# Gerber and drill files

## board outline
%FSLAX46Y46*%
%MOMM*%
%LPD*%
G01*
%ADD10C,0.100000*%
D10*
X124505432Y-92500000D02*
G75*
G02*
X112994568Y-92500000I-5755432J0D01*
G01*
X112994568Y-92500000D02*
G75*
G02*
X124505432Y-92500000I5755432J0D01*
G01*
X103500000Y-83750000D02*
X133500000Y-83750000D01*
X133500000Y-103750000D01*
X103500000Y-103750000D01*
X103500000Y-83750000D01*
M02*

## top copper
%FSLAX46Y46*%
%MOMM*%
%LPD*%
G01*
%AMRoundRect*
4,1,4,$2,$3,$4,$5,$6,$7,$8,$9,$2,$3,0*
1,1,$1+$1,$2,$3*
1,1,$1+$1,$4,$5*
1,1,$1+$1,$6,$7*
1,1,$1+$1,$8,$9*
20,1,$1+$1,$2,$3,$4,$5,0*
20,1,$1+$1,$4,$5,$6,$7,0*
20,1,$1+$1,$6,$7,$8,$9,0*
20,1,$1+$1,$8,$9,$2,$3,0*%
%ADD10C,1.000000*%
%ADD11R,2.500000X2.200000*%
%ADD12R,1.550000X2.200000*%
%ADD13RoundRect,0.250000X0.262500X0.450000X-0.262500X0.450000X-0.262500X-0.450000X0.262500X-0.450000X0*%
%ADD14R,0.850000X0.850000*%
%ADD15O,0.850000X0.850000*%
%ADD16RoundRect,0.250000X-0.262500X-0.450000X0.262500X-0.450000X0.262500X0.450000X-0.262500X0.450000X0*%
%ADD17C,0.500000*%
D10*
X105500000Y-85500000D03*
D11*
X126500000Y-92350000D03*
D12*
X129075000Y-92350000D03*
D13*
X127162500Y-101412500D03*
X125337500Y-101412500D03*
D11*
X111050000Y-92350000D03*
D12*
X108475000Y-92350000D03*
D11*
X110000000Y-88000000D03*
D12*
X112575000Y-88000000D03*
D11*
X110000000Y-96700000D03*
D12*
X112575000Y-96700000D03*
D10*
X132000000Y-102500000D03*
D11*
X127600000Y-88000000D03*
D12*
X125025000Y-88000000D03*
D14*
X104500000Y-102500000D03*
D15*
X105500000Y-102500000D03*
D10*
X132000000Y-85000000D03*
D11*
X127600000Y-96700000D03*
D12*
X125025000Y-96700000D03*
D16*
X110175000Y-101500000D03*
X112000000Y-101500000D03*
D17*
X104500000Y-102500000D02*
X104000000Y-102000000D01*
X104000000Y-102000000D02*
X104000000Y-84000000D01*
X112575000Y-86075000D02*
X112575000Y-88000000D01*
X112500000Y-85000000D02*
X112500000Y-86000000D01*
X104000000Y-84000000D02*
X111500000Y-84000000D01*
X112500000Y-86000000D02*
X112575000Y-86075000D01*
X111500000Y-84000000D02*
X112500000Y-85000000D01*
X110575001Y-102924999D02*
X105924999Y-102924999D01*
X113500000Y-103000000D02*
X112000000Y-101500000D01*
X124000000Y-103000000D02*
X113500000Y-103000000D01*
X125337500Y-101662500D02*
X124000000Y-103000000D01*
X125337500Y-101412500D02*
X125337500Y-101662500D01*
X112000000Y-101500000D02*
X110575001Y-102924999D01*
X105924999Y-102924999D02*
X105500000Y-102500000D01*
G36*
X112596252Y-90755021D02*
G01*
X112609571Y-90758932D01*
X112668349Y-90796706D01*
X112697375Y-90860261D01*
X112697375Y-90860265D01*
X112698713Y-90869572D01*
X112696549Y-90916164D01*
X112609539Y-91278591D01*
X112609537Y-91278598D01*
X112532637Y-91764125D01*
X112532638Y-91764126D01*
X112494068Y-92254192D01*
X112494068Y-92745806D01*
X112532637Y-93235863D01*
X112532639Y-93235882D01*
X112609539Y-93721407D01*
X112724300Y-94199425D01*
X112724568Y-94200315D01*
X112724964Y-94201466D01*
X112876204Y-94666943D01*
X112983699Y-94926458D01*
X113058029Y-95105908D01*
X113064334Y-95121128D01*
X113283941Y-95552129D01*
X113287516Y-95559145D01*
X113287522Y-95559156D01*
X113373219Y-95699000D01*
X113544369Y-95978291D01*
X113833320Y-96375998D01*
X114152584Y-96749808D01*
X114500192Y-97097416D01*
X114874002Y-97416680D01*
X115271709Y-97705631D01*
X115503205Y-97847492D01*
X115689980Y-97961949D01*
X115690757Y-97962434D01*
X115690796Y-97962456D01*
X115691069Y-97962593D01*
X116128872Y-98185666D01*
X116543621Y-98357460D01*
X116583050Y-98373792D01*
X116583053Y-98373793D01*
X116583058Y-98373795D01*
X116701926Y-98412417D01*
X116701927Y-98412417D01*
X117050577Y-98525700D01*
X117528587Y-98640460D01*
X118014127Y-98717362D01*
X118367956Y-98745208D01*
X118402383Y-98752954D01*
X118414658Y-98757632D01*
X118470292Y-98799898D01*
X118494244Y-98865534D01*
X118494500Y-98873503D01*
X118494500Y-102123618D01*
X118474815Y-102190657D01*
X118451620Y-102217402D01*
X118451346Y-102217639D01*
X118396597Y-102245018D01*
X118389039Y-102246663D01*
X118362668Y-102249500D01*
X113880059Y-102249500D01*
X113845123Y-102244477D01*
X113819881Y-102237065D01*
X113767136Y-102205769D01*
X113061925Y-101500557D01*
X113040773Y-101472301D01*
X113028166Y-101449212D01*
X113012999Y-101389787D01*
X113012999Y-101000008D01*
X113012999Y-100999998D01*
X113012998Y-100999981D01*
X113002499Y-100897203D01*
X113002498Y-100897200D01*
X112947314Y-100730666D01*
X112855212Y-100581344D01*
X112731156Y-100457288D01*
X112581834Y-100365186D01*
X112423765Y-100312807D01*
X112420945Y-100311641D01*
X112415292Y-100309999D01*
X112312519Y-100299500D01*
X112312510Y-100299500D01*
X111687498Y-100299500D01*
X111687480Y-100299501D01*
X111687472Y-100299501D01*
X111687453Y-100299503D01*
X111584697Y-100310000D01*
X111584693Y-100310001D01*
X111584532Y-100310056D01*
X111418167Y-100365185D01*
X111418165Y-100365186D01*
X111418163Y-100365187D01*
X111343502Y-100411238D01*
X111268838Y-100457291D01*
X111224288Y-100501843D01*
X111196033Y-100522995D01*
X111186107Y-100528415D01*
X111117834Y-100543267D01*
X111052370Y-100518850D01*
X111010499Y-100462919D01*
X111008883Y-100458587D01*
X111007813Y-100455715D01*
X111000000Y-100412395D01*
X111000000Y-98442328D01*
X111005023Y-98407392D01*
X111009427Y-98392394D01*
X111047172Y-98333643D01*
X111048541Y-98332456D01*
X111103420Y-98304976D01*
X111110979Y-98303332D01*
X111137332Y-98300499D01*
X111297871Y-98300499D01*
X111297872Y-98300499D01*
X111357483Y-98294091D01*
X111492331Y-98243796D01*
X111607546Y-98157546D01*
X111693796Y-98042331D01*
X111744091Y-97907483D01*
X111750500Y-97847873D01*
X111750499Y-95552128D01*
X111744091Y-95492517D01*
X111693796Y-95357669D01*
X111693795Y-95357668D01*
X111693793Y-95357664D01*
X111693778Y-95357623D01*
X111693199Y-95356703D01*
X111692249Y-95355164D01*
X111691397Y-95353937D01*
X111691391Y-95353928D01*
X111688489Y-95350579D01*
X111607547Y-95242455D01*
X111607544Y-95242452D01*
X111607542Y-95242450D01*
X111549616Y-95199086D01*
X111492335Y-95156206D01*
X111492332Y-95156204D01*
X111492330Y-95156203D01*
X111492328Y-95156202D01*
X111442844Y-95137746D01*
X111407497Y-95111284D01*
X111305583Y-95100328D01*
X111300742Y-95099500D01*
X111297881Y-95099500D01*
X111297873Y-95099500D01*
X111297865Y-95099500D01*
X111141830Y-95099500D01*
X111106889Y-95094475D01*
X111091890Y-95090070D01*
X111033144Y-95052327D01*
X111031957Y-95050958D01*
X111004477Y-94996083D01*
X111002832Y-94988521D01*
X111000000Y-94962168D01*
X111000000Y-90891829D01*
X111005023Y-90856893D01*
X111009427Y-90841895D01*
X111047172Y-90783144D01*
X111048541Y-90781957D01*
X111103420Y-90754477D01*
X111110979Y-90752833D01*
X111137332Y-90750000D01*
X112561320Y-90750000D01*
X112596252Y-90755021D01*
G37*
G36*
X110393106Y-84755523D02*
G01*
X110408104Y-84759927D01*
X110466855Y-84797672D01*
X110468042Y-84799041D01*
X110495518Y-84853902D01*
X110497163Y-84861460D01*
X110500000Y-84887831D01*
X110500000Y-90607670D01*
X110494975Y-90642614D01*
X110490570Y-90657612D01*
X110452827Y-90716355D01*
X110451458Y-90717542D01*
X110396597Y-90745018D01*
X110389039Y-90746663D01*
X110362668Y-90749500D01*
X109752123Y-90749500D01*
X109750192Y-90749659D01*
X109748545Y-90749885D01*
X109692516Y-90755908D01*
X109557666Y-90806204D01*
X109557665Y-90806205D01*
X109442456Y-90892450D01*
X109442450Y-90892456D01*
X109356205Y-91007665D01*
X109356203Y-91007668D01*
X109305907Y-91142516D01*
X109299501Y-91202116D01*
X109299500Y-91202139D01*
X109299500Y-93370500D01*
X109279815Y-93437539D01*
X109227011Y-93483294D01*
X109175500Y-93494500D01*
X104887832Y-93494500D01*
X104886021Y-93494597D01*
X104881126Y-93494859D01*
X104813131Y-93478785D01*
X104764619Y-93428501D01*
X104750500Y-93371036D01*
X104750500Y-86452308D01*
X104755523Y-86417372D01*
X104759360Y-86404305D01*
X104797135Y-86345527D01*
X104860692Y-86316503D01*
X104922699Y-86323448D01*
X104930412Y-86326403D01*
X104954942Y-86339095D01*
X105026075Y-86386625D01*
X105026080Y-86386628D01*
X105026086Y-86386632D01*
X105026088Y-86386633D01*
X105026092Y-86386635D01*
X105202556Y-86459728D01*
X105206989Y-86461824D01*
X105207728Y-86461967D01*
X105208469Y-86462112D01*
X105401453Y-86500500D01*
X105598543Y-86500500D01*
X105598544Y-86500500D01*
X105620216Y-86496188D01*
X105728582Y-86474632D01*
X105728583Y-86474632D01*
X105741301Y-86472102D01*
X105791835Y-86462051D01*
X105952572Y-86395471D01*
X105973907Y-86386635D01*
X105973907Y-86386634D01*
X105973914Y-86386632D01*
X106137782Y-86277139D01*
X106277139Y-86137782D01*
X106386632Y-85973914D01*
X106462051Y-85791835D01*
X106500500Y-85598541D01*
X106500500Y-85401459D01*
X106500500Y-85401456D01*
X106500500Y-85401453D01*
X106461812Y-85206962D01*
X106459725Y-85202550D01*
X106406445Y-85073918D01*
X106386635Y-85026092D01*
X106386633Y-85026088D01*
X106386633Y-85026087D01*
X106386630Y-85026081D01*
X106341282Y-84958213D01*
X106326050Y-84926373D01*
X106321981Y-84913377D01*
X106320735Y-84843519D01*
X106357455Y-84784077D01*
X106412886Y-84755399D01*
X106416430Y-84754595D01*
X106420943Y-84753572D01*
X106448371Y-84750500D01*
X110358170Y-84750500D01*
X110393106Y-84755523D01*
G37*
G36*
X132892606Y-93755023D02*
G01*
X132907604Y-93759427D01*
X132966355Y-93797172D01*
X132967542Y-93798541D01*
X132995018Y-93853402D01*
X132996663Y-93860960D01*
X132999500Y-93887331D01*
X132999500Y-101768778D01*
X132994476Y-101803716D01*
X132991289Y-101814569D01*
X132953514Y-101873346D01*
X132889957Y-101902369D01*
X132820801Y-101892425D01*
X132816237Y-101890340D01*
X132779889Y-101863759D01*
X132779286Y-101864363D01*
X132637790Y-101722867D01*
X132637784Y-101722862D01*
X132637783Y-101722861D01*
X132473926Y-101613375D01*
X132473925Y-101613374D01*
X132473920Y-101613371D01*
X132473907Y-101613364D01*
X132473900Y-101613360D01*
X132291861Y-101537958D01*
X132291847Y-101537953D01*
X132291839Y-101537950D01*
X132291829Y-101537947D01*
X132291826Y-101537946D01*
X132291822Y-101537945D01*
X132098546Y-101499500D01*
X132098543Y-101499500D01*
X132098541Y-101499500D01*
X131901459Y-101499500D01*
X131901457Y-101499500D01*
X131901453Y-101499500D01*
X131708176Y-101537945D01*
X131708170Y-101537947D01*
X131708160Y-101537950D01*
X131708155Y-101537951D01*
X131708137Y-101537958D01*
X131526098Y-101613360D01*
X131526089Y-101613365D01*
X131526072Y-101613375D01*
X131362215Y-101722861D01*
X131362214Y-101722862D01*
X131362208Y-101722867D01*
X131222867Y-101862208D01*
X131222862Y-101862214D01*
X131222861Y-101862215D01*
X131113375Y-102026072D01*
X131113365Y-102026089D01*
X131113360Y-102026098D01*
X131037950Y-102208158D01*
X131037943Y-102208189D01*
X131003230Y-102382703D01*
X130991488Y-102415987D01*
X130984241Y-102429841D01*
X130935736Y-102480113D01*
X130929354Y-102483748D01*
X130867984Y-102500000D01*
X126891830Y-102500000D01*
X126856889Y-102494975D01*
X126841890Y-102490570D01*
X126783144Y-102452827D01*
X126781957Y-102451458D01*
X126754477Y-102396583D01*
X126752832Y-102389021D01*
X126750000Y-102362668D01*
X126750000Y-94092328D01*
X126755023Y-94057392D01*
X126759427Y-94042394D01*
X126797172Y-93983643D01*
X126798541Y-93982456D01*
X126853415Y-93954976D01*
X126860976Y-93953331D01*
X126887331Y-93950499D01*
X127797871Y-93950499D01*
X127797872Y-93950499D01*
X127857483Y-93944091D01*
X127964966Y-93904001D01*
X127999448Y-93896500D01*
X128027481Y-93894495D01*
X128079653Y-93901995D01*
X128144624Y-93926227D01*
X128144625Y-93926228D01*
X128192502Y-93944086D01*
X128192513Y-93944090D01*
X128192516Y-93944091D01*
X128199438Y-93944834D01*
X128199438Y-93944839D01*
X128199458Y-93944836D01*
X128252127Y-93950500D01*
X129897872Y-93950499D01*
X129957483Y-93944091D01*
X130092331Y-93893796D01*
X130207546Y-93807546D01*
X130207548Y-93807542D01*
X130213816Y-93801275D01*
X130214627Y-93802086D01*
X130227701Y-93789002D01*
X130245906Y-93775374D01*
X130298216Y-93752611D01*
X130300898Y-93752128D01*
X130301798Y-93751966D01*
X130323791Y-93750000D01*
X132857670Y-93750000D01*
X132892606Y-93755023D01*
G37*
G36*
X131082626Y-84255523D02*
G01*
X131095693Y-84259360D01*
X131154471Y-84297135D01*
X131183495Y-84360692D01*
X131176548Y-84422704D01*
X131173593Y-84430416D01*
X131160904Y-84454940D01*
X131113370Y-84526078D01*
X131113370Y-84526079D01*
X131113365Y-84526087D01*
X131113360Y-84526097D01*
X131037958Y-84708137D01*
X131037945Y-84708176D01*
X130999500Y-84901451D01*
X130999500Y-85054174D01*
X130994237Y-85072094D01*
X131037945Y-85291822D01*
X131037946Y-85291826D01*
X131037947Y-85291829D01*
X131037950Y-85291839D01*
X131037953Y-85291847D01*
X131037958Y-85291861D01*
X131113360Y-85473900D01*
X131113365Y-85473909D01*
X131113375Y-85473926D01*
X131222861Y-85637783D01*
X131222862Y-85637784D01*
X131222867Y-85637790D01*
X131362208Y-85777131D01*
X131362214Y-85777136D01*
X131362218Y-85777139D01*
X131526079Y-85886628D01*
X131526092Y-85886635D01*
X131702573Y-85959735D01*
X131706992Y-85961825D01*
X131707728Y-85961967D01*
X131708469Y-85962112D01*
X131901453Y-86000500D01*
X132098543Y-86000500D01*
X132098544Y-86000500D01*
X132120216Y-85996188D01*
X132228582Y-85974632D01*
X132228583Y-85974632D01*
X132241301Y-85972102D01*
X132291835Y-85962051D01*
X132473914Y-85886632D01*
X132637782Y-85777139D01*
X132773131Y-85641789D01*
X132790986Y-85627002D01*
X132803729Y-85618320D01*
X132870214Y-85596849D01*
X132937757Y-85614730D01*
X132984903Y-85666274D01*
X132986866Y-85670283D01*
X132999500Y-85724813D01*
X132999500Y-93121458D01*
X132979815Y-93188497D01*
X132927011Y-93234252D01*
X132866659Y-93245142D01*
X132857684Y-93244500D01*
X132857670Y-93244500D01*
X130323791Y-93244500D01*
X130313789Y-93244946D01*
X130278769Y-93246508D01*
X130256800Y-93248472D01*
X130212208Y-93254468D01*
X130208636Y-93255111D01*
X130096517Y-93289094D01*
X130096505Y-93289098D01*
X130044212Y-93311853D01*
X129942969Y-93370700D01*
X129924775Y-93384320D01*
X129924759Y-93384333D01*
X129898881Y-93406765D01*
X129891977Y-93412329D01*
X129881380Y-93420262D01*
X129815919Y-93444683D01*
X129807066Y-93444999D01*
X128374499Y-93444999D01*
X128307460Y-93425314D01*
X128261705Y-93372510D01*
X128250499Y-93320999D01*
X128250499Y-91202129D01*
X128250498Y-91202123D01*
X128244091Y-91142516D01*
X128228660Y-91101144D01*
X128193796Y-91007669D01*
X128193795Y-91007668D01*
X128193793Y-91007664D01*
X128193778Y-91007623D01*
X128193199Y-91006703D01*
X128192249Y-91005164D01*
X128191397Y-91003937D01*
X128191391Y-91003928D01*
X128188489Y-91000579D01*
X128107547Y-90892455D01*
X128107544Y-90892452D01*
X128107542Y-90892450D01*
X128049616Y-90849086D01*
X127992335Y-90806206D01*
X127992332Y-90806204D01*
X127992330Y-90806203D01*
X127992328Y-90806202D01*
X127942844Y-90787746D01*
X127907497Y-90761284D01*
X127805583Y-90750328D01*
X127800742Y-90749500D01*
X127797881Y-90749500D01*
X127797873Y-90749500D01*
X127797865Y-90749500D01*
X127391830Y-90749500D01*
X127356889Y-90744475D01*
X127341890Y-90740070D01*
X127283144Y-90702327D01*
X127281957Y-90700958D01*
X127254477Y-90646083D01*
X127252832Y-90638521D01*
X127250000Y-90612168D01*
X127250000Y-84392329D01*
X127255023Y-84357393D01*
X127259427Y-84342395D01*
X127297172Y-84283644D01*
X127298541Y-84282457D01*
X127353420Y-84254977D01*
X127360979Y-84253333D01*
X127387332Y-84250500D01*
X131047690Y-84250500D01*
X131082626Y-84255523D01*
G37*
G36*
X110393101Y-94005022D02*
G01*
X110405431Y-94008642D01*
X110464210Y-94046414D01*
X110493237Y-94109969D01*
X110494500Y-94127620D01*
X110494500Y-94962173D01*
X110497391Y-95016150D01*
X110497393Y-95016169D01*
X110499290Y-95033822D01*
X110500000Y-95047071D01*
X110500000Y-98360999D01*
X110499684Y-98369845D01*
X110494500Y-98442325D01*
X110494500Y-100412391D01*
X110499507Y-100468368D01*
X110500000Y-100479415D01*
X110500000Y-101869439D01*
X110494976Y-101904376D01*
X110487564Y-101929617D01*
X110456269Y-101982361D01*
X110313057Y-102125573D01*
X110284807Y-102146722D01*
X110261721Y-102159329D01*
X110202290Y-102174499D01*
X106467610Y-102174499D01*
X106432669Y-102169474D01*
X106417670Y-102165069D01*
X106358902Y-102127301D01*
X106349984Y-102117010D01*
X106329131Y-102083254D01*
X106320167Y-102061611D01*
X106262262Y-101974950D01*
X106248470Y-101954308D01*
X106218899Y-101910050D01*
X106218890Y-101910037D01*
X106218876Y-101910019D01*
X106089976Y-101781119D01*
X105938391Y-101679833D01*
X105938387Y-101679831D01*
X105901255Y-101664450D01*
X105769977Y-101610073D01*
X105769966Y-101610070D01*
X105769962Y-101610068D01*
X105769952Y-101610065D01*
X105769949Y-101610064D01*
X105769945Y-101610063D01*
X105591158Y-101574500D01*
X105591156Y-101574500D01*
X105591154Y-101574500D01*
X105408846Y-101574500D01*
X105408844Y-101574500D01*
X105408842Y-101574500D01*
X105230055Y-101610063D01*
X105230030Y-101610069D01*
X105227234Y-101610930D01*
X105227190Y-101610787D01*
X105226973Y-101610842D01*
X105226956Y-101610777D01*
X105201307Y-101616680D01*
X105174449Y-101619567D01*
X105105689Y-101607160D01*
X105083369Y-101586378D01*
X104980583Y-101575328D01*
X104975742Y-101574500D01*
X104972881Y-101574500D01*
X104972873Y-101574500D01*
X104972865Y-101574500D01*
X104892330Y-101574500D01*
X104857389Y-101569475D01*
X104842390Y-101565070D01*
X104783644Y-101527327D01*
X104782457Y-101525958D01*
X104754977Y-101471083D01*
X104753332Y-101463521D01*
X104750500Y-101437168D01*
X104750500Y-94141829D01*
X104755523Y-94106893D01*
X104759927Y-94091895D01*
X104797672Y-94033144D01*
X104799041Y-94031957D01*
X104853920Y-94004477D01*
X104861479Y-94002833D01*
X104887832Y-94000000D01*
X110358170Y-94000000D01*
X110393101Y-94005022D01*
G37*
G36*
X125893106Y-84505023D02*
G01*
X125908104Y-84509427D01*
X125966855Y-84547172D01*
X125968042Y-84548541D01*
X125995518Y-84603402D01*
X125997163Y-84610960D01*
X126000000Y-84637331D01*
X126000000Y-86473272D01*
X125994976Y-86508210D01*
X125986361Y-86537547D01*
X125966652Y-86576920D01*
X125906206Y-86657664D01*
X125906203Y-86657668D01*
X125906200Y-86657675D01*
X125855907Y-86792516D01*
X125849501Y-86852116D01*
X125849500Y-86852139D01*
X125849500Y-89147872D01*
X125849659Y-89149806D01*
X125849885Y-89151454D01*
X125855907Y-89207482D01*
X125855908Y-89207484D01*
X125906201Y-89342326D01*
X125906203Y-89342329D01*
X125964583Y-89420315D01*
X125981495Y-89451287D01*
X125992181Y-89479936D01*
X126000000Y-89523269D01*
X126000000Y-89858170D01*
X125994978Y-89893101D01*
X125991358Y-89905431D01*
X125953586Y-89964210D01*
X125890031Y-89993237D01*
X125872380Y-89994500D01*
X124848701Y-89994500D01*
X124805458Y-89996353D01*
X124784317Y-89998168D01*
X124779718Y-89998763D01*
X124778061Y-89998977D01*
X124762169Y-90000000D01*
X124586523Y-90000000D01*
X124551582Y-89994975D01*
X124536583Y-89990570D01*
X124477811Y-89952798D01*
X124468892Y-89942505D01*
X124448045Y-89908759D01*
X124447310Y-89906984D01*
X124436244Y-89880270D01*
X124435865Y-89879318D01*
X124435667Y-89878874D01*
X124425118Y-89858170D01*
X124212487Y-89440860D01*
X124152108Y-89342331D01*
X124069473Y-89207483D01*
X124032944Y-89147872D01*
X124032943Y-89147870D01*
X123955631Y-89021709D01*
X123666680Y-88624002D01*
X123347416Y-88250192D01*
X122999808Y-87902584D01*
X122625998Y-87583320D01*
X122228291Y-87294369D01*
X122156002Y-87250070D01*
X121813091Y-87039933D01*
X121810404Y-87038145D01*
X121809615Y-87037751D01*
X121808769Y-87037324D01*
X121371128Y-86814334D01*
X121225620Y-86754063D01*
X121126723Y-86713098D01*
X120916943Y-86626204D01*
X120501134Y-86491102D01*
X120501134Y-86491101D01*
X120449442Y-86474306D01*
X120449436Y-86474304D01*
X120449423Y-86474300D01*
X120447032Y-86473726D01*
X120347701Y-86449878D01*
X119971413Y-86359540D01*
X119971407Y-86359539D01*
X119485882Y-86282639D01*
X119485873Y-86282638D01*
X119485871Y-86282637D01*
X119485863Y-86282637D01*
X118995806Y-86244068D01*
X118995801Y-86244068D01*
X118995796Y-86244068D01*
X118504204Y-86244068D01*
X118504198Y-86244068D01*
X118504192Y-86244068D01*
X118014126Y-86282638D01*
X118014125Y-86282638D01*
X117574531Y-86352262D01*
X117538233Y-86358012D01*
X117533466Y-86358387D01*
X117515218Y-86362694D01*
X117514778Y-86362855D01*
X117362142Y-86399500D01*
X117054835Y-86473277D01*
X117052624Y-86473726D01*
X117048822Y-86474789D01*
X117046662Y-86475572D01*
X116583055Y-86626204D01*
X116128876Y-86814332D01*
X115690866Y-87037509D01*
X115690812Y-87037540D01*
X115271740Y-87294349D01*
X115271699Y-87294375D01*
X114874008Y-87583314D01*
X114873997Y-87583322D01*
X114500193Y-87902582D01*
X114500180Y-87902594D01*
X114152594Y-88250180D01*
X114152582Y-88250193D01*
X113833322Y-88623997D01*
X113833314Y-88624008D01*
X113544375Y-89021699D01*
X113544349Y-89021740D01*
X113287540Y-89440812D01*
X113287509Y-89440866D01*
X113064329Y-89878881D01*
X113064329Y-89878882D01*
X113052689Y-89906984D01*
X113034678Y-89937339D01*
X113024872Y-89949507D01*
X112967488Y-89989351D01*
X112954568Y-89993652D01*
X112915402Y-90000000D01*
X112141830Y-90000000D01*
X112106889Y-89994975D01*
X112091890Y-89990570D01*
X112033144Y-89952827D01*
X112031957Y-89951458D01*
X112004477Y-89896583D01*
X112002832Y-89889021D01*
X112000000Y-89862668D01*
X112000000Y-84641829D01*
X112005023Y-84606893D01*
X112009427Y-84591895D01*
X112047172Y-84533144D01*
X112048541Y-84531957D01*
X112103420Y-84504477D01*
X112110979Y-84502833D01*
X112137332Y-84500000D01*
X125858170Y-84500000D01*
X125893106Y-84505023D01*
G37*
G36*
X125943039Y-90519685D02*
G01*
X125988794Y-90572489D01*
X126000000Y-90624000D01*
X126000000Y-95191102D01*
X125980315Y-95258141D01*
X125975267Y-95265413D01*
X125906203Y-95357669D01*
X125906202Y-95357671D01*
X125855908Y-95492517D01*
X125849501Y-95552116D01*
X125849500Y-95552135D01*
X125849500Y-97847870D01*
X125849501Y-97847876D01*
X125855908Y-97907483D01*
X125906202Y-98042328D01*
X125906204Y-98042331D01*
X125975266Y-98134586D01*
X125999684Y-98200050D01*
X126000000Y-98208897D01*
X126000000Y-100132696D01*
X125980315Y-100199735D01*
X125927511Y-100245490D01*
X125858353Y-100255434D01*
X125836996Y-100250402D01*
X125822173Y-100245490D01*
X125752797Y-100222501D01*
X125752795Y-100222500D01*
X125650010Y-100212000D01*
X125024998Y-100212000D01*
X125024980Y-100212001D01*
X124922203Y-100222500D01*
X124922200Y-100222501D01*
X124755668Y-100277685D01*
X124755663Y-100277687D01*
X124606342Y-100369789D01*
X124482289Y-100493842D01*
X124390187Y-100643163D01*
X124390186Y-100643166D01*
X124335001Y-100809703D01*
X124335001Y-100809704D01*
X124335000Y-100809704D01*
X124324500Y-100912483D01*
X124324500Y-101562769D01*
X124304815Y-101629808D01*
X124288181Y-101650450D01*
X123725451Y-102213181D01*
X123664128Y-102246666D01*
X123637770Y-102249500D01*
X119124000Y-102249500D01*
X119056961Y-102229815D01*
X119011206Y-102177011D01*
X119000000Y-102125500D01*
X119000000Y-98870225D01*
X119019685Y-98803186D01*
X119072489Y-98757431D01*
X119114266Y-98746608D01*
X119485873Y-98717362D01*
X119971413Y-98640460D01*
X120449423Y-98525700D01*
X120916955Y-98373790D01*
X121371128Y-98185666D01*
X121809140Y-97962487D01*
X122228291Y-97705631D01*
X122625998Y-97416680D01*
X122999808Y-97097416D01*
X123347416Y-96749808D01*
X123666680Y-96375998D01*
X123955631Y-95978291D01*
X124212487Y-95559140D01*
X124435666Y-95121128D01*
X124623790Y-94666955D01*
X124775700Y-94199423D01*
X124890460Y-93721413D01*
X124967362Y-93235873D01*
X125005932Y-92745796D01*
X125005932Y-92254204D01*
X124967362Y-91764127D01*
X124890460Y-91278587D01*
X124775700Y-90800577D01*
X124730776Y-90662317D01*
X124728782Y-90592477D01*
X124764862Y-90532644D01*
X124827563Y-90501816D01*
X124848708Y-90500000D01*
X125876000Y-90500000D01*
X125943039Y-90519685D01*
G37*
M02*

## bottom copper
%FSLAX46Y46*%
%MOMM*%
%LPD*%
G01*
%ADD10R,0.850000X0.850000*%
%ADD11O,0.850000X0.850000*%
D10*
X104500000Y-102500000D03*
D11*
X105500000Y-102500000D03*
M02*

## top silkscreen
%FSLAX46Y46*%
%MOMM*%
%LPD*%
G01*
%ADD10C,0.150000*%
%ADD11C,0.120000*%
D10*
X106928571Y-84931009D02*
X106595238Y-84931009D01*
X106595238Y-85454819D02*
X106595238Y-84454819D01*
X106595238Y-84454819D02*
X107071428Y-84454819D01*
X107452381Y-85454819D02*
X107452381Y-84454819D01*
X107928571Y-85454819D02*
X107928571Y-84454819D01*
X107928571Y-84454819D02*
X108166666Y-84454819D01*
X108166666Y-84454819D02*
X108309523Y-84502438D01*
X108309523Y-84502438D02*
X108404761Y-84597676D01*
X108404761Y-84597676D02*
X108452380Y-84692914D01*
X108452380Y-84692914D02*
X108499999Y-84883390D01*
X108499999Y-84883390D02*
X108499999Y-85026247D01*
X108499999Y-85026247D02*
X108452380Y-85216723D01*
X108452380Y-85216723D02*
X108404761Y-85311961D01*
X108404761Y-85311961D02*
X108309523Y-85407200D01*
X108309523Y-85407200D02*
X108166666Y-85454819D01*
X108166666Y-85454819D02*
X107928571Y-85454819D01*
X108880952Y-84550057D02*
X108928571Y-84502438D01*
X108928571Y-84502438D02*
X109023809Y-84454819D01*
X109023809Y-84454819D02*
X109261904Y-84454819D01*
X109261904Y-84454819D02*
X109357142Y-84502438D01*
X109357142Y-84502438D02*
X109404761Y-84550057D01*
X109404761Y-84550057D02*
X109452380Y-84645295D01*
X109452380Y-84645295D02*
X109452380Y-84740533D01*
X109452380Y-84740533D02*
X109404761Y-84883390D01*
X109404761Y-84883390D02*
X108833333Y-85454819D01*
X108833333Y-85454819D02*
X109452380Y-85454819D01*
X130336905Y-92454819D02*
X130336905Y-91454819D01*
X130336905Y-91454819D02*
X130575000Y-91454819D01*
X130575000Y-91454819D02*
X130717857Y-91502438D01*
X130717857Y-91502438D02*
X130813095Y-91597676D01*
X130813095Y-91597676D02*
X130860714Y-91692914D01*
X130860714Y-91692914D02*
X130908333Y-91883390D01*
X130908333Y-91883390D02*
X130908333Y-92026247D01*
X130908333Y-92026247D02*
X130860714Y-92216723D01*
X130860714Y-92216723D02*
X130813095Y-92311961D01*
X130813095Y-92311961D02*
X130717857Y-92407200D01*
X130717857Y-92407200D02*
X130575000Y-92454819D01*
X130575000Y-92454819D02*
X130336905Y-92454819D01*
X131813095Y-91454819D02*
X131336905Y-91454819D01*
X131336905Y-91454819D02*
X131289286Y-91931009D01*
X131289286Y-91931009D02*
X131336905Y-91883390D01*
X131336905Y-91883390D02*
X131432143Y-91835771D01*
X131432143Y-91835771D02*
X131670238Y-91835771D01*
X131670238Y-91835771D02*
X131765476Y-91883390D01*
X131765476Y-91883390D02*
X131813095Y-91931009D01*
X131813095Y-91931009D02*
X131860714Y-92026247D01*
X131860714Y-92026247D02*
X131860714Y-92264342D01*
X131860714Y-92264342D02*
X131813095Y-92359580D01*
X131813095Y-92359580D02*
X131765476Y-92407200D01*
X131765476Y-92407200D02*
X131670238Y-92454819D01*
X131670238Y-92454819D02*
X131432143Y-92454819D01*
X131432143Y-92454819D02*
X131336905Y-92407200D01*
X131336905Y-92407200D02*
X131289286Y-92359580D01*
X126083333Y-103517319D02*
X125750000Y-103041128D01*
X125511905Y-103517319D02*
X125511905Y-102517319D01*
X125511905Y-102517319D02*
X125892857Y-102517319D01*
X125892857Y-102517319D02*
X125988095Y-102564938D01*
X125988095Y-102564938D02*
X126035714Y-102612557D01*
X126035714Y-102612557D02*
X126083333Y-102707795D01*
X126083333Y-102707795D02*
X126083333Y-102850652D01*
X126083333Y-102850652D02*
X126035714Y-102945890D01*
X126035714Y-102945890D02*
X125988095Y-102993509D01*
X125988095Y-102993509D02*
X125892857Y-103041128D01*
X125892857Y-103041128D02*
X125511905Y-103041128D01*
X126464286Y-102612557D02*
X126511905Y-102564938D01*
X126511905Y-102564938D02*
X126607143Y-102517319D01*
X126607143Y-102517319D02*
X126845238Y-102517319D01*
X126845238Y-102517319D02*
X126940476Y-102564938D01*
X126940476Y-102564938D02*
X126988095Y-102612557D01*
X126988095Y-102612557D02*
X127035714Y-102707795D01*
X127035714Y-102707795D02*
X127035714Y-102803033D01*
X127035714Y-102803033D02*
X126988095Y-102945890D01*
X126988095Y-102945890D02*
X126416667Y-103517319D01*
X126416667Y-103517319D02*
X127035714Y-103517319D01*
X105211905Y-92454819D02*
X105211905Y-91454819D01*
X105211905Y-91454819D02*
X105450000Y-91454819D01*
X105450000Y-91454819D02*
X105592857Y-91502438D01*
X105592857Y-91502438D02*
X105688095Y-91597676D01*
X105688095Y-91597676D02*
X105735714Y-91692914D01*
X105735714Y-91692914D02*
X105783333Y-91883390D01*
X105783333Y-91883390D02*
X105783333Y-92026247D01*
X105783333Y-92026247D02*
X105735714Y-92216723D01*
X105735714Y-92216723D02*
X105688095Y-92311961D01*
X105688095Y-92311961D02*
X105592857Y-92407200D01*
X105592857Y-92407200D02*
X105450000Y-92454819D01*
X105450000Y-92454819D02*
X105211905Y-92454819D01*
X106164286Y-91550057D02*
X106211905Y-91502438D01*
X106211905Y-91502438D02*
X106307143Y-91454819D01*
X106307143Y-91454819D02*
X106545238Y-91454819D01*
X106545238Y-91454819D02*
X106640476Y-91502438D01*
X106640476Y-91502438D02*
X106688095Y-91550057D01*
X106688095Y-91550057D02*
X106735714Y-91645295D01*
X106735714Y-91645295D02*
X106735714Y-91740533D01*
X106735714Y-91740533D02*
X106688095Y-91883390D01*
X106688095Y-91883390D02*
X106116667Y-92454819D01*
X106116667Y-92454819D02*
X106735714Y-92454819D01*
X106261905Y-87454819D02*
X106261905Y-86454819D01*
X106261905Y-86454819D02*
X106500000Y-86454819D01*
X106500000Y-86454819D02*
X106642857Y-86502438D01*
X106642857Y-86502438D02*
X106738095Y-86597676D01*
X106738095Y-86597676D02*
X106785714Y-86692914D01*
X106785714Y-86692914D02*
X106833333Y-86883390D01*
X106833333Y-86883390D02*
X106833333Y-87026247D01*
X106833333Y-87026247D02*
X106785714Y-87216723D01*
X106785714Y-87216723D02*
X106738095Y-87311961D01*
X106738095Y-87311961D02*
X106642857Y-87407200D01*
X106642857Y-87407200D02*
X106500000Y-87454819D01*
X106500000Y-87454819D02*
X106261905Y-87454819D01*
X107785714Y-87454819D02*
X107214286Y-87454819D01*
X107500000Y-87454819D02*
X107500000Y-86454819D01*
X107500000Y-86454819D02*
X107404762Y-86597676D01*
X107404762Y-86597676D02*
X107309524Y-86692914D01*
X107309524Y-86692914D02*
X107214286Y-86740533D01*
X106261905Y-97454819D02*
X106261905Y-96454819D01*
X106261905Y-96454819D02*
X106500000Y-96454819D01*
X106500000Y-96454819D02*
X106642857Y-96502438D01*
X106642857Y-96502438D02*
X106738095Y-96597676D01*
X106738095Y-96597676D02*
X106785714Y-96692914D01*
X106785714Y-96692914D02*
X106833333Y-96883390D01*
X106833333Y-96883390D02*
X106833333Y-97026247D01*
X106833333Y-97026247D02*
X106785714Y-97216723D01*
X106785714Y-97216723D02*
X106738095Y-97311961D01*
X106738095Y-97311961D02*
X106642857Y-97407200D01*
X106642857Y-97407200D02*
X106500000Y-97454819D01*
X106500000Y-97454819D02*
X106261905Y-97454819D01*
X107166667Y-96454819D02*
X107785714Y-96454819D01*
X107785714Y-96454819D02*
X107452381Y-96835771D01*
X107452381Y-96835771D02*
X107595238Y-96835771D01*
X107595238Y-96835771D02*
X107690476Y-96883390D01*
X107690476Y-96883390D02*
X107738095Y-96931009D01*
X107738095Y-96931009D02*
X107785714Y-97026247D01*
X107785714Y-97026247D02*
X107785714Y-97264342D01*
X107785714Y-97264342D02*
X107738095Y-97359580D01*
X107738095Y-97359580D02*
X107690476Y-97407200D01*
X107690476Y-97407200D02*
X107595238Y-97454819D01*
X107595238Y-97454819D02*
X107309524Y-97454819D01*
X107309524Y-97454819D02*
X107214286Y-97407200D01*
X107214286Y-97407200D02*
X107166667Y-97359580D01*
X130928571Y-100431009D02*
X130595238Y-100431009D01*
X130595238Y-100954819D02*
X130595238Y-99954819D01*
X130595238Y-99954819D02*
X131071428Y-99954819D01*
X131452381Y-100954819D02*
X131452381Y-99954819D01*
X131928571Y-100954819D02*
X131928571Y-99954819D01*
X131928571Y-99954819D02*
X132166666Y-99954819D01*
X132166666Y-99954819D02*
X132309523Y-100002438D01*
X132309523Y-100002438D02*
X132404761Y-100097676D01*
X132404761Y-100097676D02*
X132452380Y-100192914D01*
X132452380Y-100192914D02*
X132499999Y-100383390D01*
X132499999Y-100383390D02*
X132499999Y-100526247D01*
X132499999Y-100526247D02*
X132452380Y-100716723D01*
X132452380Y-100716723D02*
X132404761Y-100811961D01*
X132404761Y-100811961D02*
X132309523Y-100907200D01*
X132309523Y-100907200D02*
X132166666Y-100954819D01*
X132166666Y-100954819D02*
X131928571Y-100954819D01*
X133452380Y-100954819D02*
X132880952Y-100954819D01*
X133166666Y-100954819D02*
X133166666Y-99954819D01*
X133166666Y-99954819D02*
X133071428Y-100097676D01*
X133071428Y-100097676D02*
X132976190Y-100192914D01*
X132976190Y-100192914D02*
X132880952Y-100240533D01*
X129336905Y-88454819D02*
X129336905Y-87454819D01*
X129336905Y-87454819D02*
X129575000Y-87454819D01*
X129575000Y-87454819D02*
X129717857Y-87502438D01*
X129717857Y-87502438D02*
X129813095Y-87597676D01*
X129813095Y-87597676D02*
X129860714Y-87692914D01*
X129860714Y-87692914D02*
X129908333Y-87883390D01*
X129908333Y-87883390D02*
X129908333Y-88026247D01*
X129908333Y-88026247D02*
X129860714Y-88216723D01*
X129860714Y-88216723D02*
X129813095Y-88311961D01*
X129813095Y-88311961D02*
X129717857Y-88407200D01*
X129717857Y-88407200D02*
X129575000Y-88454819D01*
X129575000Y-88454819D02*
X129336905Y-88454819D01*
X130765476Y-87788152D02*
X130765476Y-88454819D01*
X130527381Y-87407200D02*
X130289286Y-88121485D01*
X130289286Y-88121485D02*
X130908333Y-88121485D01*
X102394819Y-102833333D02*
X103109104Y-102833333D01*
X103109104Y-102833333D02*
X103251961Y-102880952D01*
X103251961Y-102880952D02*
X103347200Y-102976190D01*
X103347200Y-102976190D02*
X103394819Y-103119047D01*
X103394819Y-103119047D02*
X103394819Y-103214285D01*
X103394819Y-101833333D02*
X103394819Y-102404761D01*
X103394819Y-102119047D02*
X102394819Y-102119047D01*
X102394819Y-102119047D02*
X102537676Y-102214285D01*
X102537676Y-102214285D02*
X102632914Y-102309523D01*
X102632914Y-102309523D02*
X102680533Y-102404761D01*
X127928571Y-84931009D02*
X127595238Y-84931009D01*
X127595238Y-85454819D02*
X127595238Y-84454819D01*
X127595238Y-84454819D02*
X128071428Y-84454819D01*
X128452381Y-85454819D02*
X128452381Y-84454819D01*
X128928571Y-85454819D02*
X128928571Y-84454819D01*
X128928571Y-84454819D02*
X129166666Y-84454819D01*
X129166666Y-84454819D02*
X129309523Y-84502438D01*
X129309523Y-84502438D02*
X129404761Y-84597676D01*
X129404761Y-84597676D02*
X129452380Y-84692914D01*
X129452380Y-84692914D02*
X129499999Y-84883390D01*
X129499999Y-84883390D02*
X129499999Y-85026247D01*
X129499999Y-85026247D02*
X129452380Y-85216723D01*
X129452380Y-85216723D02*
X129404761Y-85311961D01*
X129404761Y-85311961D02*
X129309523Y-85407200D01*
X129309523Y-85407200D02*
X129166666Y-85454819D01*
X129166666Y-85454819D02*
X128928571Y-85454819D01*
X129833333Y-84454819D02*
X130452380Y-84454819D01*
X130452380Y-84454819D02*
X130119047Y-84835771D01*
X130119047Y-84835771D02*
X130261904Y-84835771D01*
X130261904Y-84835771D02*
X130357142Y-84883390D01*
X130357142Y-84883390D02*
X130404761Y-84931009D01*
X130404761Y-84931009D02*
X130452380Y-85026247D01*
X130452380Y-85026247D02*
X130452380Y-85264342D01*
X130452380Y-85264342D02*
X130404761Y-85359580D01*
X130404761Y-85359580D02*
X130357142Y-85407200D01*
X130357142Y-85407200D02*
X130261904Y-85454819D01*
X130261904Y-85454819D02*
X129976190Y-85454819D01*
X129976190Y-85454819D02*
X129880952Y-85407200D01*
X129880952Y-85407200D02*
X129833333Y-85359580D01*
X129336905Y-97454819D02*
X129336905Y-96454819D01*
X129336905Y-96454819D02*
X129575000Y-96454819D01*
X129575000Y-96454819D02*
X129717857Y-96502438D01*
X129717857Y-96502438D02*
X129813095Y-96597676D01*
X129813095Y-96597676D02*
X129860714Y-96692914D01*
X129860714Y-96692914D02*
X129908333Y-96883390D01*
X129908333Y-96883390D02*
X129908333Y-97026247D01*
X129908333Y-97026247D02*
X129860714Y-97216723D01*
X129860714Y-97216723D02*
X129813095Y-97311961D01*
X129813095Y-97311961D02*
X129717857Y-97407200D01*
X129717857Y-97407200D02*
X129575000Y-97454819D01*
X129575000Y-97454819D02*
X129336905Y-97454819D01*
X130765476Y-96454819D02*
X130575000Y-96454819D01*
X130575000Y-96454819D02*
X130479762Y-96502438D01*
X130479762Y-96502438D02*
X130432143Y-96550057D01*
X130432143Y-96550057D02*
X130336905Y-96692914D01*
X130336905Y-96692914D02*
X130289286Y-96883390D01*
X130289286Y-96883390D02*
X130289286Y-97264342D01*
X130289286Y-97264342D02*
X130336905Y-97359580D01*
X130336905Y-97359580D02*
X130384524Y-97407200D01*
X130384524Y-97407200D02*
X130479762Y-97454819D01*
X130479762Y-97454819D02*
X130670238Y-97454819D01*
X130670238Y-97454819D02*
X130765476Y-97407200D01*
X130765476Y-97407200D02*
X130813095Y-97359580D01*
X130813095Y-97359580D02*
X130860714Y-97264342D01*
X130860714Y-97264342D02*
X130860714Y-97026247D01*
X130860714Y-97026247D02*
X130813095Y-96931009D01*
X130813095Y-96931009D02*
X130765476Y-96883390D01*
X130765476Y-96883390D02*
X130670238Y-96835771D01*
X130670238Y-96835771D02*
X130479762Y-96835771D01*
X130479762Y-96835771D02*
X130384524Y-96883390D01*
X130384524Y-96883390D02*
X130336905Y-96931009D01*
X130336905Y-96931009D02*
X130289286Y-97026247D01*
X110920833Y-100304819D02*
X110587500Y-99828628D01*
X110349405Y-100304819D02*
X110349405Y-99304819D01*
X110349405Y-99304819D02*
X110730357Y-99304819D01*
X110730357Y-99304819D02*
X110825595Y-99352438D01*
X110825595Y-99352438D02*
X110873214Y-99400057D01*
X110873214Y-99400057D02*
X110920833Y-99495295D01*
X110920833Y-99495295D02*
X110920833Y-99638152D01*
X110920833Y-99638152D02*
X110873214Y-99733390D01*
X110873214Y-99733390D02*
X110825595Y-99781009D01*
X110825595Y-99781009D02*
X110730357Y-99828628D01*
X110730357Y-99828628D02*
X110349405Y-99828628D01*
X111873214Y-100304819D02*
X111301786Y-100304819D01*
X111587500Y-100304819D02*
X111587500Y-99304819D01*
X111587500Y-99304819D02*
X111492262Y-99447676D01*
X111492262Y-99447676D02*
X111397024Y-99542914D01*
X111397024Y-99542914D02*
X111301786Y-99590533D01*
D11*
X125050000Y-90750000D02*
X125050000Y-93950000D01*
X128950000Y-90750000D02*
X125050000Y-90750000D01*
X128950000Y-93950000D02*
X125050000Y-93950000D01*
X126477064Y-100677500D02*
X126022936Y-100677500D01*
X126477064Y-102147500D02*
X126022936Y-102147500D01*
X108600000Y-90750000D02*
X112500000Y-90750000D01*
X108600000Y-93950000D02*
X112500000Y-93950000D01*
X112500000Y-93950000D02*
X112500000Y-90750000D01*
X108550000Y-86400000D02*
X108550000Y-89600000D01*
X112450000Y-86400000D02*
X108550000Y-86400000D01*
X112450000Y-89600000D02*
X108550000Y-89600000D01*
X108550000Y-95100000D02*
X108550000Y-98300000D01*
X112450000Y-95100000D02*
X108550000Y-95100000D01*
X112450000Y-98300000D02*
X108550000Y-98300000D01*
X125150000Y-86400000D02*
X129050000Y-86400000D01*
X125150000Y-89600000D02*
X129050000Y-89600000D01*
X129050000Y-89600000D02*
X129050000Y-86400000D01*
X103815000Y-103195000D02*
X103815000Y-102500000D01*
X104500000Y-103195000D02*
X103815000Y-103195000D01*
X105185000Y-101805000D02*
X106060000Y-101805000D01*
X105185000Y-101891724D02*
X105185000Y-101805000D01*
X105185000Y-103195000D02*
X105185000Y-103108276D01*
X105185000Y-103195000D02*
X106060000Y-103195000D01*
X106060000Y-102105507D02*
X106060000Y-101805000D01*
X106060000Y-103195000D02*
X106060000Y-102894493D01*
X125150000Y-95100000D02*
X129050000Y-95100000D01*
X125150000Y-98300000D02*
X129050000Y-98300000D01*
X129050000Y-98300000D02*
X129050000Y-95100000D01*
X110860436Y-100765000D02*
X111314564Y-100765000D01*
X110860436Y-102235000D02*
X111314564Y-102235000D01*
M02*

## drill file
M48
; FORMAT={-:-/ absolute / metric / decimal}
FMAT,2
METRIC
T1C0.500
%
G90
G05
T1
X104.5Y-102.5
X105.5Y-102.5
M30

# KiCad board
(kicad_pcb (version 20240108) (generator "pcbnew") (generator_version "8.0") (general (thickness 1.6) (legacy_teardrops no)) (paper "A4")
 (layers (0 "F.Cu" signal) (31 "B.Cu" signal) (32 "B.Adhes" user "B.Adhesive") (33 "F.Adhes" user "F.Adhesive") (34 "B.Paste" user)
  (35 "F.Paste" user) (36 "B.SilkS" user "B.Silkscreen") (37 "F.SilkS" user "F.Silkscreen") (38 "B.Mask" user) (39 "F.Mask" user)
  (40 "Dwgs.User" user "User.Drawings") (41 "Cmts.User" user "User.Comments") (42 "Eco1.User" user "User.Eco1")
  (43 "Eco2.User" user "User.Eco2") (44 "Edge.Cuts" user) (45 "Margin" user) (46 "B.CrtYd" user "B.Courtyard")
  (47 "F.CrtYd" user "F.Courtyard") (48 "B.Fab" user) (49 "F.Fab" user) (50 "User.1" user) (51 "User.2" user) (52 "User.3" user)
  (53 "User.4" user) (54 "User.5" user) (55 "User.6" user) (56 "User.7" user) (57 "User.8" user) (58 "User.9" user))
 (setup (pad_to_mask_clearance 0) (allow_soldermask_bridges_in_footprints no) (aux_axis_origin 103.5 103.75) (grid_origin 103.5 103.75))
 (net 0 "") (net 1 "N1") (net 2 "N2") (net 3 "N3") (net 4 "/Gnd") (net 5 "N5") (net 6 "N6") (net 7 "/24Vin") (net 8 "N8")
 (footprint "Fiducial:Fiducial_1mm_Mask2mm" (layer "F.Cu") (at 105.5 85.5)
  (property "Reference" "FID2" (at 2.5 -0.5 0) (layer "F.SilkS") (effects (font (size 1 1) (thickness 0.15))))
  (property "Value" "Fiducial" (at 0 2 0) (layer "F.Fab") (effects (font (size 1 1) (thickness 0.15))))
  (pad "" smd circle (at 0 0) (size 1 1) (layers "F.Cu" "F.Mask") (solder_mask_margin 0.5) (clearance 0.5)))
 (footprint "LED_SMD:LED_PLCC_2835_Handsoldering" (layer "F.Cu") (at 127.55 92.35)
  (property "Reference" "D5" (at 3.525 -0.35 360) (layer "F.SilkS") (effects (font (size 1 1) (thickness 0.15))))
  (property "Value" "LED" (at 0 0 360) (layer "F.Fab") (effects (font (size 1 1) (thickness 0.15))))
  (fp_line (start -2.5 -1.6) (end -2.5 1.6) (stroke (width 0.12) (type solid)) (layer "F.SilkS"))
  (fp_line (start 1.4 -1.6) (end -2.5 -1.6) (stroke (width 0.12) (type solid)) (layer "F.SilkS"))
  (fp_line (start 1.4 1.6) (end -2.5 1.6) (stroke (width 0.12) (type solid)) (layer "F.SilkS"))
  (pad "1" smd rect (at -1.05 0) (size 2.5 2.2) (layers "F.Cu" "F.Paste" "F.Mask") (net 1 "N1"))
  (pad "2" smd rect (at 1.525 0) (size 1.55 2.2) (layers "F.Cu" "F.Paste" "F.Mask") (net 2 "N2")))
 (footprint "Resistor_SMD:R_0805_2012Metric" (layer "F.Cu") (at 126.25 101.4125 180)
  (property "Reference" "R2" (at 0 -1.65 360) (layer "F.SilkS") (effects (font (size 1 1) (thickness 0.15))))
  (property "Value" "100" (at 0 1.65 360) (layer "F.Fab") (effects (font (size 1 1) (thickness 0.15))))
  (fp_line (start -0.227064 0.735) (end 0.227064 0.735) (stroke (width 0.12) (type solid)) (layer "F.SilkS"))
  (fp_line (start -0.227064 -0.735) (end 0.227064 -0.735) (stroke (width 0.12) (type solid)) (layer "F.SilkS"))
  (pad "1" smd roundrect (at -0.9125 0 180) (size 1.025 1.4) (layers "F.Cu" "F.Paste" "F.Mask") (roundrect_rratio 0.243902) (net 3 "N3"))
  (pad "2" smd roundrect (at 0.9125 0 180) (size 1.025 1.4) (layers "F.Cu" "F.Paste" "F.Mask") (roundrect_rratio 0.243902) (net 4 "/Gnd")))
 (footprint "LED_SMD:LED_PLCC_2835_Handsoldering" (layer "F.Cu") (at 110 92.35 180)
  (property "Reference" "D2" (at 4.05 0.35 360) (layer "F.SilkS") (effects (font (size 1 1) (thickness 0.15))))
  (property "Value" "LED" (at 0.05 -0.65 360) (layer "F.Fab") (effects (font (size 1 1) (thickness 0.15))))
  (fp_line (start 1.4 1.6) (end -2.5 1.6) (stroke (width 0.12) (type solid)) (layer "F.SilkS"))
  (fp_line (start 1.4 -1.6) (end -2.5 -1.6) (stroke (width 0.12) (type solid)) (layer "F.SilkS"))
  (fp_line (start -2.5 -1.6) (end -2.5 1.6) (stroke (width 0.12) (type solid)) (layer "F.SilkS"))
  (pad "1" smd rect (at -1.05 0 180) (size 2.5 2.2) (layers "F.Cu" "F.Paste" "F.Mask") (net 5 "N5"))
  (pad "2" smd rect (at 1.525 0 180) (size 1.55 2.2) (layers "F.Cu" "F.Paste" "F.Mask") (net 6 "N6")))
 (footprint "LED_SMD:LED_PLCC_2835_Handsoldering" (layer "F.Cu") (at 111.05 88)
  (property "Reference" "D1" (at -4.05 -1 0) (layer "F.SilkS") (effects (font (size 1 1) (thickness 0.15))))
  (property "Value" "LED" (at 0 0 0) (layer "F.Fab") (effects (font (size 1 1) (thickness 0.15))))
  (fp_line (start -2.5 -1.6) (end -2.5 1.6) (stroke (width 0.12) (type solid)) (layer "F.SilkS"))
  (fp_line (start 1.4 -1.6) (end -2.5 -1.6) (stroke (width 0.12) (type solid)) (layer "F.SilkS"))
  (fp_line (start 1.4 1.6) (end -2.5 1.6) (stroke (width 0.12) (type solid)) (layer "F.SilkS"))
  (pad "1" smd rect (at -1.05 0) (size 2.5 2.2) (layers "F.Cu" "F.Paste" "F.Mask") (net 6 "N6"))
  (pad "2" smd rect (at 1.525 0) (size 1.55 2.2) (layers "F.Cu" "F.Paste" "F.Mask") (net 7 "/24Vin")))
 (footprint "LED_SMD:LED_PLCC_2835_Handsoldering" (layer "F.Cu") (at 111.05 96.7)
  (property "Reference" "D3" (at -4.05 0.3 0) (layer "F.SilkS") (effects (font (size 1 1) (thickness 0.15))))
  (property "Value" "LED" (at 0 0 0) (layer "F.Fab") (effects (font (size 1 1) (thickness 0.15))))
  (fp_line (start -2.5 -1.6) (end -2.5 1.6) (stroke (width 0.12) (type solid)) (layer "F.SilkS"))
  (fp_line (start 1.4 -1.6) (end -2.5 -1.6) (stroke (width 0.12) (type solid)) (layer "F.SilkS"))
  (fp_line (start 1.4 1.6) (end -2.5 1.6) (stroke (width 0.12) (type solid)) (layer "F.SilkS"))
  (pad "1" smd rect (at -1.05 0) (size 2.5 2.2) (layers "F.Cu" "F.Paste" "F.Mask") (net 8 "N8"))
  (pad "2" smd rect (at 1.525 0) (size 1.55 2.2) (layers "F.Cu" "F.Paste" "F.Mask") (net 5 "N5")))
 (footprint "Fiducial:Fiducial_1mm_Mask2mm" (layer "F.Cu") (at 132 102.5)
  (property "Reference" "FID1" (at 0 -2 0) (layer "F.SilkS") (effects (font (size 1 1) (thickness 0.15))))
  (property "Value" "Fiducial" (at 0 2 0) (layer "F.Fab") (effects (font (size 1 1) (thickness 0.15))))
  (pad "" smd circle (at 0 0) (size 1 1) (layers "F.Cu" "F.Mask") (solder_mask_margin 0.5) (clearance 0.5)))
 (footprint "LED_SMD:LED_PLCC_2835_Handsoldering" (layer "F.Cu") (at 126.55 88 180)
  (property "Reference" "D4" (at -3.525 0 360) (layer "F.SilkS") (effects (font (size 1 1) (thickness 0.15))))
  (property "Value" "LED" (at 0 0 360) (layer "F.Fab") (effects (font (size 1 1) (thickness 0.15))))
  (fp_line (start 1.4 1.6) (end -2.5 1.6) (stroke (width 0.12) (type solid)) (layer "F.SilkS"))
  (fp_line (start 1.4 -1.6) (end -2.5 -1.6) (stroke (width 0.12) (type solid)) (layer "F.SilkS"))
  (fp_line (start -2.5 -1.6) (end -2.5 1.6) (stroke (width 0.12) (type solid)) (layer "F.SilkS"))
  (pad "1" smd rect (at -1.05 0 180) (size 2.5 2.2) (layers "F.Cu" "F.Paste" "F.Mask") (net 2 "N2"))
  (pad "2" smd rect (at 1.525 0 180) (size 1.55 2.2) (layers "F.Cu" "F.Paste" "F.Mask") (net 7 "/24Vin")))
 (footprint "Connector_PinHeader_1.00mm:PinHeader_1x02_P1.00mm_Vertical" (layer "F.Cu") (at 104.5 102.5 90)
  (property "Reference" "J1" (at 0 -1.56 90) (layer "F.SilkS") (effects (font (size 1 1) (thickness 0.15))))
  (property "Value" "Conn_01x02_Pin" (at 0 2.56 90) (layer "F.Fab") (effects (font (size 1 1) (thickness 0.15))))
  (fp_line (start -0.695 -0.685) (end 0 -0.685) (stroke (width 0.12) (type solid)) (layer "F.SilkS"))
  (fp_line (start -0.695 0) (end -0.695 -0.685) (stroke (width 0.12) (type solid)) (layer "F.SilkS"))
  (fp_line (start 0.695 0.685) (end 0.695 1.56) (stroke (width 0.12) (type solid)) (layer "F.SilkS"))
  (fp_line (start 0.608276 0.685) (end 0.695 0.685) (stroke (width 0.12) (type solid)) (layer "F.SilkS"))
  (fp_line (start -0.695 0.685) (end -0.608276 0.685) (stroke (width 0.12) (type solid)) (layer "F.SilkS"))
  (fp_line (start -0.695 0.685) (end -0.695 1.56) (stroke (width 0.12) (type solid)) (layer "F.SilkS"))
  (fp_line (start 0.394493 1.56) (end 0.695 1.56) (stroke (width 0.12) (type solid)) (layer "F.SilkS"))
  (fp_line (start -0.695 1.56) (end -0.394493 1.56) (stroke (width 0.12) (type solid)) (layer "F.SilkS"))
  (pad "1" thru_hole rect (at 0 0 90) (size 0.85 0.85) (drill 0.5) (layers "*.Cu" "*.Mask") (remove_unused_layers no) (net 7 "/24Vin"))
  (pad "2" thru_hole oval (at 0 1 90) (size 0.85 0.85) (drill 0.5) (layers "*.Cu" "*.Mask") (remove_unused_layers no) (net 4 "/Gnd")))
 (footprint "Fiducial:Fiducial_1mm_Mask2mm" (layer "F.Cu") (at 132 85)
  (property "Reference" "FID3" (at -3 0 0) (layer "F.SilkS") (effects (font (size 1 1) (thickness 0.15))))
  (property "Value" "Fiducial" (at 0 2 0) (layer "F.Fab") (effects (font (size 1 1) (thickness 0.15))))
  (pad "" smd circle (at 0 0) (size 1 1) (layers "F.Cu" "F.Mask") (solder_mask_margin 0.5) (clearance 0.5)))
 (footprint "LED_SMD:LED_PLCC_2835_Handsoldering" (layer "F.Cu") (at 126.55 96.7 180)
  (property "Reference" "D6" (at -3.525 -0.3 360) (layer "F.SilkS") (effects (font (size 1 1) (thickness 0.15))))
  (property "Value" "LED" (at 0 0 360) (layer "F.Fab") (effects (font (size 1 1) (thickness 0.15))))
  (fp_line (start 1.4 1.6) (end -2.5 1.6) (stroke (width 0.12) (type solid)) (layer "F.SilkS"))
  (fp_line (start 1.4 -1.6) (end -2.5 -1.6) (stroke (width 0.12) (type solid)) (layer "F.SilkS"))
  (fp_line (start -2.5 -1.6) (end -2.5 1.6) (stroke (width 0.12) (type solid)) (layer "F.SilkS"))
  (pad "1" smd rect (at -1.05 0 180) (size 2.5 2.2) (layers "F.Cu" "F.Paste" "F.Mask") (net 3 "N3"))
  (pad "2" smd rect (at 1.525 0 180) (size 1.55 2.2) (layers "F.Cu" "F.Paste" "F.Mask") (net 1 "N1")))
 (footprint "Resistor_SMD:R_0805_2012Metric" (layer "F.Cu") (at 111.0875 101.5)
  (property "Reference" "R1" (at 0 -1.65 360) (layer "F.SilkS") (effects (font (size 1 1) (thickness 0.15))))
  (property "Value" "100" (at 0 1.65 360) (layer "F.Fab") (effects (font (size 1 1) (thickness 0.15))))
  (fp_line (start -0.227064 -0.735) (end 0.227064 -0.735) (stroke (width 0.12) (type solid)) (layer "F.SilkS"))
  (fp_line (start -0.227064 0.735) (end 0.227064 0.735) (stroke (width 0.12) (type solid)) (layer "F.SilkS"))
  (pad "1" smd roundrect (at -0.9125 0) (size 1.025 1.4) (layers "F.Cu" "F.Paste" "F.Mask") (roundrect_rratio 0.243902) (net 8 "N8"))
  (pad "2" smd roundrect (at 0.9125 0) (size 1.025 1.4) (layers "F.Cu" "F.Paste" "F.Mask") (roundrect_rratio 0.243902) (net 4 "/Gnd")))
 (gr_circle (center 118.75 92.5) (end 124.5 92.25) (stroke (width 0.1) (type default)) (fill none) (layer "Edge.Cuts"))
 (gr_rect (start 103.5 83.75) (end 133.5 103.75) (stroke (width 0.1) (type default)) (fill none) (layer "Edge.Cuts"))
 (segment (start 104.5 102.5) (end 104 102) (width 0.5) (layer "F.Cu") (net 7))
 (segment (start 104 102) (end 104 84) (width 0.5) (layer "F.Cu") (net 7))
 (segment (start 112.575 86.075) (end 112.575 88) (width 0.5) (layer "F.Cu") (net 7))
 (segment (start 112.5 85) (end 112.5 86) (width 0.5) (layer "F.Cu") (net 7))
 (segment (start 104 84) (end 111.5 84) (width 0.5) (layer "F.Cu") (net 7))
 (segment (start 112.5 86) (end 112.575 86.075) (width 0.5) (layer "F.Cu") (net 7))
 (segment (start 111.5 84) (end 112.5 85) (width 0.5) (layer "F.Cu") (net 7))
 (segment (start 110.575001 102.924999) (end 105.924999 102.924999) (width 0.5) (layer "F.Cu") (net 4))
 (segment (start 113.5 103) (end 112 101.5) (width 0.5) (layer "F.Cu") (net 4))
 (segment (start 124 103) (end 113.5 103) (width 0.5) (layer "F.Cu") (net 4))
 (segment (start 125.3375 101.6625) (end 124 103) (width 0.5) (layer "F.Cu") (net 4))
 (segment (start 125.3375 101.4125) (end 125.3375 101.6625) (width 0.5) (layer "F.Cu") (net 4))
 (segment (start 112 101.5) (end 110.575001 102.924999) (width 0.5) (layer "F.Cu") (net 4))
 (segment (start 105.924999 102.924999) (end 105.5 102.5) (width 0.5) (layer "F.Cu") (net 4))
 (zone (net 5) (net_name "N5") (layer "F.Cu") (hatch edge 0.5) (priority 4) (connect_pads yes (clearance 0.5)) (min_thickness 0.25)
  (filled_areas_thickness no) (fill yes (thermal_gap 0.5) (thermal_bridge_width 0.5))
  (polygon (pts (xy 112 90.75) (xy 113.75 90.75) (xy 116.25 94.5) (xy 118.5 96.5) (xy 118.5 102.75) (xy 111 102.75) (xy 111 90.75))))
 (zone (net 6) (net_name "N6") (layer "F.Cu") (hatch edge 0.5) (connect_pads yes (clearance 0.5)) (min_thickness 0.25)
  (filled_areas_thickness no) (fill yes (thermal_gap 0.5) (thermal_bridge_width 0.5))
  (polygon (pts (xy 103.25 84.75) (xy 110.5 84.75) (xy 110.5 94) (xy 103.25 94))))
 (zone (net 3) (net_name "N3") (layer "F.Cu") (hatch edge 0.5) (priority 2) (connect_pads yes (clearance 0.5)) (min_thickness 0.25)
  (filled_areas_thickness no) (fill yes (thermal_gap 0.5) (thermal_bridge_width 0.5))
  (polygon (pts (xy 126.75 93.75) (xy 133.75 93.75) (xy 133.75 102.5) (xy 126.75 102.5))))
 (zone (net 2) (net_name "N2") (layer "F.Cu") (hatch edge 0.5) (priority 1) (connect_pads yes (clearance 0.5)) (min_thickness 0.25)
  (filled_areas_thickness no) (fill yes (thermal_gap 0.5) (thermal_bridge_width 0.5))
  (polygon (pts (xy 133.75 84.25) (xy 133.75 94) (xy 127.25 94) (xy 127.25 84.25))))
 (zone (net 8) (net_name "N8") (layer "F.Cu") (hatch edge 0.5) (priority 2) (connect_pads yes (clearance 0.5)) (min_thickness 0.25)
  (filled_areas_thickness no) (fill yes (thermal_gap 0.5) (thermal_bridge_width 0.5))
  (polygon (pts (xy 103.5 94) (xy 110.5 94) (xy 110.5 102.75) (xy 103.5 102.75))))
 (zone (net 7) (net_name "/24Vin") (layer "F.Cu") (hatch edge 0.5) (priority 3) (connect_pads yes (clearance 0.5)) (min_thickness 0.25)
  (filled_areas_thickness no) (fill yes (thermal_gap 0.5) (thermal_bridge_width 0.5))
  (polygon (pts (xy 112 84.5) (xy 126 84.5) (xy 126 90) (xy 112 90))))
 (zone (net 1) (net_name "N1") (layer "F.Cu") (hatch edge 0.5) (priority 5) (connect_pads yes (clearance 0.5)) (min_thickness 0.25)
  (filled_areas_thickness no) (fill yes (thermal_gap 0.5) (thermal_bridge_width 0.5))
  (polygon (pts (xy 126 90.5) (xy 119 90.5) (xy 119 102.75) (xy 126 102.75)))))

